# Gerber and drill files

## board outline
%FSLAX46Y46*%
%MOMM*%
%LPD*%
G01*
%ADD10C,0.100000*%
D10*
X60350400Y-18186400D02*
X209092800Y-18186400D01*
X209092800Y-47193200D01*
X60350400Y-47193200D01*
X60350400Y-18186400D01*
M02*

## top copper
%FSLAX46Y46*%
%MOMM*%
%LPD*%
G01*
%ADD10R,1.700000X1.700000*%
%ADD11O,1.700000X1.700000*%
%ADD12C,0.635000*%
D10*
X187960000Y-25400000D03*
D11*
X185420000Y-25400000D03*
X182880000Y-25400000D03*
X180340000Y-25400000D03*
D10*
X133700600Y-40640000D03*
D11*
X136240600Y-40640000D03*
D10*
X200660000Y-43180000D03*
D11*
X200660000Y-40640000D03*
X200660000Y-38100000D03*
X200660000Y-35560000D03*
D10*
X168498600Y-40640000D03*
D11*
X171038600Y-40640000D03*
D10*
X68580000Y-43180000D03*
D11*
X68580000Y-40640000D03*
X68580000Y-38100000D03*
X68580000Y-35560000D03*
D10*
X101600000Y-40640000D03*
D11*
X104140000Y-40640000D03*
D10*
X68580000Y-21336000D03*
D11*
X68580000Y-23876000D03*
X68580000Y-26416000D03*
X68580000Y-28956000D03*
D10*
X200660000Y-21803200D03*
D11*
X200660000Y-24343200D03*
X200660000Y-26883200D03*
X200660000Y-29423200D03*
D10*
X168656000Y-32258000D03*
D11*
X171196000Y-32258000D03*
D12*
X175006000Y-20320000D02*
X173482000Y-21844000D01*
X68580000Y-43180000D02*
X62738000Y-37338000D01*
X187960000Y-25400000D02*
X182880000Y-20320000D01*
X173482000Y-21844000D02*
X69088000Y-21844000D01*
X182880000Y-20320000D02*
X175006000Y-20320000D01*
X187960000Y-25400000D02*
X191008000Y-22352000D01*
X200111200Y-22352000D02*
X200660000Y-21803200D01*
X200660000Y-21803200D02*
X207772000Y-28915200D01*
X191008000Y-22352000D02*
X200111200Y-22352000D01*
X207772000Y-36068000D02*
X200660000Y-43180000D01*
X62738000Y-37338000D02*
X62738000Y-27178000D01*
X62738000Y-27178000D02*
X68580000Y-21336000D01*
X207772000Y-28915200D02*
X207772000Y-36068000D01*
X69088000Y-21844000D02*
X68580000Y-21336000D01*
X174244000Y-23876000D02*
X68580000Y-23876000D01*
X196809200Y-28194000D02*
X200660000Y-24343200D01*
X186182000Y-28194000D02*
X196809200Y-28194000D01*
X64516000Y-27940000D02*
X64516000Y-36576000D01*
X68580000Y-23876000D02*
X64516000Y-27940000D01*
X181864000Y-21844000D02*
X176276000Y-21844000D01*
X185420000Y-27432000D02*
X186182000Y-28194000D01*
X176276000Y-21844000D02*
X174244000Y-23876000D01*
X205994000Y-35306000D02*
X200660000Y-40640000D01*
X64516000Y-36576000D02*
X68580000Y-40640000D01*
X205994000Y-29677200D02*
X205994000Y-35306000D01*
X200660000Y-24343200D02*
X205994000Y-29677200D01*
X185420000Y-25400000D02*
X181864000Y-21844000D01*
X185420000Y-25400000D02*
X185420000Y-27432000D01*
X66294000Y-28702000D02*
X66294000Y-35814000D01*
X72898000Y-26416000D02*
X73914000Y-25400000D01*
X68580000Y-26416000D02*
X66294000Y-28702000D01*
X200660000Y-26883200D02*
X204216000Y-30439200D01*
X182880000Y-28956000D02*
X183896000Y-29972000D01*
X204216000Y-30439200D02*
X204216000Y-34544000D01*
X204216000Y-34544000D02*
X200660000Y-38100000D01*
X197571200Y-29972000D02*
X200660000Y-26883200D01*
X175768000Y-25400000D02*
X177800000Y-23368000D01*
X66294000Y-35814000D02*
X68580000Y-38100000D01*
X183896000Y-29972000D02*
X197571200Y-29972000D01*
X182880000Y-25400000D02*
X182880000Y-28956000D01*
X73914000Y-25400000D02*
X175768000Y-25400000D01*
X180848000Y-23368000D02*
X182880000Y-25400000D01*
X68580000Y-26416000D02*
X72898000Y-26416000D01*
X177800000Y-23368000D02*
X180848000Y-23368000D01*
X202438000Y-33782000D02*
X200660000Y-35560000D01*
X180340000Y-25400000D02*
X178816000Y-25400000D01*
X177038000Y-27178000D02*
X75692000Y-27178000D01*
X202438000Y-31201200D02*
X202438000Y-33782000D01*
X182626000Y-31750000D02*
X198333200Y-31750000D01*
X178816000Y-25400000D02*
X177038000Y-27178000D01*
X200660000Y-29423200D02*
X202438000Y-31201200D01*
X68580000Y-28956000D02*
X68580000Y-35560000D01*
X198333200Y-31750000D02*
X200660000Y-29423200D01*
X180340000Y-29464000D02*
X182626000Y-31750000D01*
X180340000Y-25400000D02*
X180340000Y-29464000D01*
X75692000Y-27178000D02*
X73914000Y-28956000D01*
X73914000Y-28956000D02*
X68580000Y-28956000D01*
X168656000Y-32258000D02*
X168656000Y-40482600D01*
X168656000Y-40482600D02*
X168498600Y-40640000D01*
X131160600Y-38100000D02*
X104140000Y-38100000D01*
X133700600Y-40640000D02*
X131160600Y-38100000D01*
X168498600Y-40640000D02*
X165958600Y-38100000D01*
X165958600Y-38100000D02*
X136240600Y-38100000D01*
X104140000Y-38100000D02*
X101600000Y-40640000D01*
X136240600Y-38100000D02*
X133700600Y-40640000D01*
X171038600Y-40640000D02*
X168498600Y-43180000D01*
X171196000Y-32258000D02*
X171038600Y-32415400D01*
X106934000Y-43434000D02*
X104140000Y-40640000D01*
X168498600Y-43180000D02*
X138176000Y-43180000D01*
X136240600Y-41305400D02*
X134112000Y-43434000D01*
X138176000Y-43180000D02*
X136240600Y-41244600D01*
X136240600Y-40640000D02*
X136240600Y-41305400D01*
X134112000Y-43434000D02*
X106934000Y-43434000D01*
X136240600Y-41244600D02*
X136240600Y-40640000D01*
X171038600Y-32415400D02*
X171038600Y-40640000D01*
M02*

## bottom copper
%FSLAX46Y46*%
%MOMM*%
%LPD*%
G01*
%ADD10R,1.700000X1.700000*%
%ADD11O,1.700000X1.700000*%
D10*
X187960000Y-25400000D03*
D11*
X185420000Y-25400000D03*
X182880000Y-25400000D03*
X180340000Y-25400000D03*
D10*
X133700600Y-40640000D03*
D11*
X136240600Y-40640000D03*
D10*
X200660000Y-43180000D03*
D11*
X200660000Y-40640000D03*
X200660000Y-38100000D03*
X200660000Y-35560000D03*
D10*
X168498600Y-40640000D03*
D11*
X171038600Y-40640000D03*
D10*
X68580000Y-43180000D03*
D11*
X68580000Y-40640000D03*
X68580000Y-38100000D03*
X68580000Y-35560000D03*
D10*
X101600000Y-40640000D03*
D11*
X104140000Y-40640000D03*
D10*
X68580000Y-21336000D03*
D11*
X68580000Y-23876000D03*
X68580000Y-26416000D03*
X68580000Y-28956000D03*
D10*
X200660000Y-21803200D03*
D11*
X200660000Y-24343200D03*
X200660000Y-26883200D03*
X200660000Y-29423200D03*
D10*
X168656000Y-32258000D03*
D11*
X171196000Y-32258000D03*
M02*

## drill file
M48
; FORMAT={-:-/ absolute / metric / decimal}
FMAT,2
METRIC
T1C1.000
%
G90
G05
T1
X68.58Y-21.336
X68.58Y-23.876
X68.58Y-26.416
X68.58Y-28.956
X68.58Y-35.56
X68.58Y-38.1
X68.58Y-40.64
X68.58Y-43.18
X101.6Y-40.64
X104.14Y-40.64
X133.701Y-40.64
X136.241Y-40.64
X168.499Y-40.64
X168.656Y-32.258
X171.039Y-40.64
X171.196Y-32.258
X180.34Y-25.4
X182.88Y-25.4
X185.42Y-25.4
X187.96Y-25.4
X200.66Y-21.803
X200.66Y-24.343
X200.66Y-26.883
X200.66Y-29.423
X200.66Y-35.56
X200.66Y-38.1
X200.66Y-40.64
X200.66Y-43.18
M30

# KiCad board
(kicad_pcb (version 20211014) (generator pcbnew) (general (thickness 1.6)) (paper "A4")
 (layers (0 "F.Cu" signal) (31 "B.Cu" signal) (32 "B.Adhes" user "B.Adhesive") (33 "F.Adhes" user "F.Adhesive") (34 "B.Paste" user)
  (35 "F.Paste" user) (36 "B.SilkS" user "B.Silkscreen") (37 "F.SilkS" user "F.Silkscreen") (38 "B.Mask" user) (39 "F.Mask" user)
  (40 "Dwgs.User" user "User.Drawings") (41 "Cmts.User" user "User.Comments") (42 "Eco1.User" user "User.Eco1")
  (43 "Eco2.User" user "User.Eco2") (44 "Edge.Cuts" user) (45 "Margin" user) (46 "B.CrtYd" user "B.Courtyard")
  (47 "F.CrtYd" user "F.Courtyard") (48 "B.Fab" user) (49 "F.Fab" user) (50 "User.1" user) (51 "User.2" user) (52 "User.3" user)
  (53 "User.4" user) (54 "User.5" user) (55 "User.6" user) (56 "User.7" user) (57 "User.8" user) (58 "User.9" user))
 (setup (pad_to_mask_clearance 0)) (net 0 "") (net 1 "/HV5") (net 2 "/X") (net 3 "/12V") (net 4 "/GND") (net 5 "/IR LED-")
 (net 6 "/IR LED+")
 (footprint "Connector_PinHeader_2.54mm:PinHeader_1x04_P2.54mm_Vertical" (layer "F.Cu") (at 187.96 25.4 -90)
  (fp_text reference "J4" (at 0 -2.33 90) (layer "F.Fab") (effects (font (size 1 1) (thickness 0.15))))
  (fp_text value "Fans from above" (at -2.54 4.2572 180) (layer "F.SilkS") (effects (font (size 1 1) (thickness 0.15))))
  (pad "1" thru_hole rect (at 0 0 270) (size 1.7 1.7) (drill 1) (layers *.Cu *.Mask) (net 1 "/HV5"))
  (pad "2" thru_hole oval (at 0 2.54 270) (size 1.7 1.7) (drill 1) (layers *.Cu *.Mask) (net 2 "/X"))
  (pad "3" thru_hole oval (at 0 5.08 270) (size 1.7 1.7) (drill 1) (layers *.Cu *.Mask) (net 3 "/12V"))
  (pad "4" thru_hole oval (at 0 7.62 270) (size 1.7 1.7) (drill 1) (layers *.Cu *.Mask) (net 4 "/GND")))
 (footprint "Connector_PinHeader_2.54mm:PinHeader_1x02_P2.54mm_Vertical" (layer "F.Cu") (at 133.7006 40.64 90)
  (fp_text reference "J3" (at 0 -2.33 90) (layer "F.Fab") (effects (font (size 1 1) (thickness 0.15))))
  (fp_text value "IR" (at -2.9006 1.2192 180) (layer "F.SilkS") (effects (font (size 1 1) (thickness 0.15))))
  (pad "1" thru_hole rect (at 0 0 90) (size 1.7 1.7) (drill 1) (layers *.Cu *.Mask) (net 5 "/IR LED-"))
  (pad "2" thru_hole oval (at 0 2.54 90) (size 1.7 1.7) (drill 1) (layers *.Cu *.Mask) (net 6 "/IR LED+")))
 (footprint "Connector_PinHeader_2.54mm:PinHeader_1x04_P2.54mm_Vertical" (layer "F.Cu") (at 200.66 43.18 180)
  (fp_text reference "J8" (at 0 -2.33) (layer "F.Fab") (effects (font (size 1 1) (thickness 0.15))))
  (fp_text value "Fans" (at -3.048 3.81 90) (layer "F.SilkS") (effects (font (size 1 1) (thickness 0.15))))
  (pad "1" thru_hole rect (at 0 0 180) (size 1.7 1.7) (drill 1) (layers *.Cu *.Mask) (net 1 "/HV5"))
  (pad "2" thru_hole oval (at 0 2.54 180) (size 1.7 1.7) (drill 1) (layers *.Cu *.Mask) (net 2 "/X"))
  (pad "3" thru_hole oval (at 0 5.08 180) (size 1.7 1.7) (drill 1) (layers *.Cu *.Mask) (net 3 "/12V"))
  (pad "4" thru_hole oval (at 0 7.62 180) (size 1.7 1.7) (drill 1) (layers *.Cu *.Mask) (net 4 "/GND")))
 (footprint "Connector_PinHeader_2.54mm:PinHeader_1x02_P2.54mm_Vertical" (layer "F.Cu") (at 168.4986 40.64 90)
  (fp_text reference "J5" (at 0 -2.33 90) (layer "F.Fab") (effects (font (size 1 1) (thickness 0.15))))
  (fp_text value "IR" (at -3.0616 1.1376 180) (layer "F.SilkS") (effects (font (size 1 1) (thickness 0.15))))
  (pad "1" thru_hole rect (at 0 0 90) (size 1.7 1.7) (drill 1) (layers *.Cu *.Mask) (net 5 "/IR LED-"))
  (pad "2" thru_hole oval (at 0 2.54 90) (size 1.7 1.7) (drill 1) (layers *.Cu *.Mask) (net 6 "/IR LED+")))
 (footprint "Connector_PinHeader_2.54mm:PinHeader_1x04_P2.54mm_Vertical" (layer "F.Cu") (at 68.58 43.18 180)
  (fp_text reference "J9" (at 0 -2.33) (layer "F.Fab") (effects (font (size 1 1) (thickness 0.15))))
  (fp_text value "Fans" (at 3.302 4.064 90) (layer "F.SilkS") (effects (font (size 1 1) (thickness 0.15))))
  (pad "1" thru_hole rect (at 0 0 180) (size 1.7 1.7) (drill 1) (layers *.Cu *.Mask) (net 1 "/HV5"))
  (pad "2" thru_hole oval (at 0 2.54 180) (size 1.7 1.7) (drill 1) (layers *.Cu *.Mask) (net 2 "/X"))
  (pad "3" thru_hole oval (at 0 5.08 180) (size 1.7 1.7) (drill 1) (layers *.Cu *.Mask) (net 3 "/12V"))
  (pad "4" thru_hole oval (at 0 7.62 180) (size 1.7 1.7) (drill 1) (layers *.Cu *.Mask) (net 4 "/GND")))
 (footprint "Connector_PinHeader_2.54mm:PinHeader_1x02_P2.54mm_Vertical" (layer "F.Cu") (at 101.6 40.64 90)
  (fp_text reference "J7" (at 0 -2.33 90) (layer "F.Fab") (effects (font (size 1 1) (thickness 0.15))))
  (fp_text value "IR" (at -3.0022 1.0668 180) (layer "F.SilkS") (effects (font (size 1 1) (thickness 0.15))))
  (pad "1" thru_hole rect (at 0 0 90) (size 1.7 1.7) (drill 1) (layers *.Cu *.Mask) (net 5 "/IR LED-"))
  (pad "2" thru_hole oval (at 0 2.54 90) (size 1.7 1.7) (drill 1) (layers *.Cu *.Mask) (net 6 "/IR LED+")))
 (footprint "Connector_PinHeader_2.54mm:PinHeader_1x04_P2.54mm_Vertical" (layer "F.Cu") (at 68.58 21.336)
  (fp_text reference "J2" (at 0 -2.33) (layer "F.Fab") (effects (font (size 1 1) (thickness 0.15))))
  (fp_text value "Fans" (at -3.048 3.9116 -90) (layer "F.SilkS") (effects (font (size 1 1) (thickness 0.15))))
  (pad "1" thru_hole rect (at 0 0) (size 1.7 1.7) (drill 1) (layers *.Cu *.Mask) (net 1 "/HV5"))
  (pad "2" thru_hole oval (at 0 2.54) (size 1.7 1.7) (drill 1) (layers *.Cu *.Mask) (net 2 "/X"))
  (pad "3" thru_hole oval (at 0 5.08) (size 1.7 1.7) (drill 1) (layers *.Cu *.Mask) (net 3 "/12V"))
  (pad "4" thru_hole oval (at 0 7.62) (size 1.7 1.7) (drill 1) (layers *.Cu *.Mask) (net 4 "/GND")))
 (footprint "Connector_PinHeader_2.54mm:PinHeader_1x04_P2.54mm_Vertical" (layer "F.Cu") (at 200.66 21.8032)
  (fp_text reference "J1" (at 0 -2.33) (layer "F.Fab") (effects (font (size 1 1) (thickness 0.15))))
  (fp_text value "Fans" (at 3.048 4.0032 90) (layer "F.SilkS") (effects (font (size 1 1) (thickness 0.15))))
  (pad "1" thru_hole rect (at 0 0) (size 1.7 1.7) (drill 1) (layers *.Cu *.Mask) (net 1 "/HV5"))
  (pad "2" thru_hole oval (at 0 2.54) (size 1.7 1.7) (drill 1) (layers *.Cu *.Mask) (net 2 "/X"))
  (pad "3" thru_hole oval (at 0 5.08) (size 1.7 1.7) (drill 1) (layers *.Cu *.Mask) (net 3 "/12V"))
  (pad "4" thru_hole oval (at 0 7.62) (size 1.7 1.7) (drill 1) (layers *.Cu *.Mask) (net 4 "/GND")))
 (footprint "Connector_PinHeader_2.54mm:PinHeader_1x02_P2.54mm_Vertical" (layer "F.Cu") (at 168.656 32.258 90)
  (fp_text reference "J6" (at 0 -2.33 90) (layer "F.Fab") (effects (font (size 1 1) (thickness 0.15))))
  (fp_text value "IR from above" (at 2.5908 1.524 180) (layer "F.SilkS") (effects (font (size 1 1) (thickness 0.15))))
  (pad "1" thru_hole rect (at 0 0 90) (size 1.7 1.7) (drill 1) (layers *.Cu *.Mask) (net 5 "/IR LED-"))
  (pad "2" thru_hole oval (at 0 2.54 90) (size 1.7 1.7) (drill 1) (layers *.Cu *.Mask) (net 6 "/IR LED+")))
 (gr_rect (start 60.3504 18.1864) (end 209.0928 47.1932) (layer "Edge.Cuts") (width 0.1) (fill none))
 (segment (start 175.006 20.32) (end 173.482 21.844) (width 0.635) (layer "F.Cu") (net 1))
 (segment (start 68.58 43.18) (end 62.738 37.338) (width 0.635) (layer "F.Cu") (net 1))
 (segment (start 187.96 25.4) (end 182.88 20.32) (width 0.635) (layer "F.Cu") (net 1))
 (segment (start 173.482 21.844) (end 69.088 21.844) (width 0.635) (layer "F.Cu") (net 1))
 (segment (start 182.88 20.32) (end 175.006 20.32) (width 0.635) (layer "F.Cu") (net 1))
 (segment (start 187.96 25.4) (end 191.008 22.352) (width 0.635) (layer "F.Cu") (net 1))
 (segment (start 200.1112 22.352) (end 200.66 21.8032) (width 0.635) (layer "F.Cu") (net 1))
 (segment (start 200.66 21.8032) (end 207.772 28.9152) (width 0.635) (layer "F.Cu") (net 1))
 (segment (start 191.008 22.352) (end 200.1112 22.352) (width 0.635) (layer "F.Cu") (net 1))
 (segment (start 207.772 36.068) (end 200.66 43.18) (width 0.635) (layer "F.Cu") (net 1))
 (segment (start 62.738 37.338) (end 62.738 27.178) (width 0.635) (layer "F.Cu") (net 1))
 (segment (start 62.738 27.178) (end 68.58 21.336) (width 0.635) (layer "F.Cu") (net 1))
 (segment (start 207.772 28.9152) (end 207.772 36.068) (width 0.635) (layer "F.Cu") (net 1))
 (segment (start 69.088 21.844) (end 68.58 21.336) (width 0.635) (layer "F.Cu") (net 1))
 (segment (start 174.244 23.876) (end 68.58 23.876) (width 0.635) (layer "F.Cu") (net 2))
 (segment (start 196.8092 28.194) (end 200.66 24.3432) (width 0.635) (layer "F.Cu") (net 2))
 (segment (start 186.182 28.194) (end 196.8092 28.194) (width 0.635) (layer "F.Cu") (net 2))
 (segment (start 64.516 27.94) (end 64.516 36.576) (width 0.635) (layer "F.Cu") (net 2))
 (segment (start 68.58 23.876) (end 64.516 27.94) (width 0.635) (layer "F.Cu") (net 2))
 (segment (start 181.864 21.844) (end 176.276 21.844) (width 0.635) (layer "F.Cu") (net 2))
 (segment (start 185.42 27.432) (end 186.182 28.194) (width 0.635) (layer "F.Cu") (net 2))
 (segment (start 176.276 21.844) (end 174.244 23.876) (width 0.635) (layer "F.Cu") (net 2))
 (segment (start 205.994 35.306) (end 200.66 40.64) (width 0.635) (layer "F.Cu") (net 2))
 (segment (start 64.516 36.576) (end 68.58 40.64) (width 0.635) (layer "F.Cu") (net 2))
 (segment (start 205.994 29.6772) (end 205.994 35.306) (width 0.635) (layer "F.Cu") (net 2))
 (segment (start 200.66 24.3432) (end 205.994 29.6772) (width 0.635) (layer "F.Cu") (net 2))
 (segment (start 185.42 25.4) (end 181.864 21.844) (width 0.635) (layer "F.Cu") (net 2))
 (segment (start 185.42 25.4) (end 185.42 27.432) (width 0.635) (layer "F.Cu") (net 2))
 (segment (start 66.294 28.702) (end 66.294 35.814) (width 0.635) (layer "F.Cu") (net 3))
 (segment (start 72.898 26.416) (end 73.914 25.4) (width 0.635) (layer "F.Cu") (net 3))
 (segment (start 68.58 26.416) (end 66.294 28.702) (width 0.635) (layer "F.Cu") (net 3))
 (segment (start 200.66 26.8832) (end 204.216 30.4392) (width 0.635) (layer "F.Cu") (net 3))
 (segment (start 182.88 28.956) (end 183.896 29.972) (width 0.635) (layer "F.Cu") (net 3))
 (segment (start 204.216 30.4392) (end 204.216 34.544) (width 0.635) (layer "F.Cu") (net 3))
 (segment (start 204.216 34.544) (end 200.66 38.1) (width 0.635) (layer "F.Cu") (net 3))
 (segment (start 197.5712 29.972) (end 200.66 26.8832) (width 0.635) (layer "F.Cu") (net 3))
 (segment (start 175.768 25.4) (end 177.8 23.368) (width 0.635) (layer "F.Cu") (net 3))
 (segment (start 66.294 35.814) (end 68.58 38.1) (width 0.635) (layer "F.Cu") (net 3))
 (segment (start 183.896 29.972) (end 197.5712 29.972) (width 0.635) (layer "F.Cu") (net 3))
 (segment (start 182.88 25.4) (end 182.88 28.956) (width 0.635) (layer "F.Cu") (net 3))
 (segment (start 73.914 25.4) (end 175.768 25.4) (width 0.635) (layer "F.Cu") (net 3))
 (segment (start 180.848 23.368) (end 182.88 25.4) (width 0.635) (layer "F.Cu") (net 3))
 (segment (start 68.58 26.416) (end 72.898 26.416) (width 0.635) (layer "F.Cu") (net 3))
 (segment (start 177.8 23.368) (end 180.848 23.368) (width 0.635) (layer "F.Cu") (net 3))
 (segment (start 202.438 33.782) (end 200.66 35.56) (width 0.635) (layer "F.Cu") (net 4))
 (segment (start 180.34 25.4) (end 178.816 25.4) (width 0.635) (layer "F.Cu") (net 4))
 (segment (start 177.038 27.178) (end 75.692 27.178) (width 0.635) (layer "F.Cu") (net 4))
 (segment (start 202.438 31.2012) (end 202.438 33.782) (width 0.635) (layer "F.Cu") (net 4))
 (segment (start 182.626 31.75) (end 198.3332 31.75) (width 0.635) (layer "F.Cu") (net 4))
 (segment (start 178.816 25.4) (end 177.038 27.178) (width 0.635) (layer "F.Cu") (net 4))
 (segment (start 200.66 29.4232) (end 202.438 31.2012) (width 0.635) (layer "F.Cu") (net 4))
 (segment (start 68.58 28.956) (end 68.58 35.56) (width 0.635) (layer "F.Cu") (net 4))
 (segment (start 198.3332 31.75) (end 200.66 29.4232) (width 0.635) (layer "F.Cu") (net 4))
 (segment (start 180.34 29.464) (end 182.626 31.75) (width 0.635) (layer "F.Cu") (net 4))
 (segment (start 180.34 25.4) (end 180.34 29.464) (width 0.635) (layer "F.Cu") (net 4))
 (segment (start 75.692 27.178) (end 73.914 28.956) (width 0.635) (layer "F.Cu") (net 4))
 (segment (start 73.914 28.956) (end 68.58 28.956) (width 0.635) (layer "F.Cu") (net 4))
 (segment (start 168.656 32.258) (end 168.656 40.4826) (width 0.635) (layer "F.Cu") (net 5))
 (segment (start 168.656 40.4826) (end 168.4986 40.64) (width 0.635) (layer "F.Cu") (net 5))
 (segment (start 131.1606 38.1) (end 104.14 38.1) (width 0.635) (layer "F.Cu") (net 5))
 (segment (start 133.7006 40.64) (end 131.1606 38.1) (width 0.635) (layer "F.Cu") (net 5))
 (segment (start 168.4986 40.64) (end 165.9586 38.1) (width 0.635) (layer "F.Cu") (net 5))
 (segment (start 165.9586 38.1) (end 136.2406 38.1) (width 0.635) (layer "F.Cu") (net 5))
 (segment (start 104.14 38.1) (end 101.6 40.64) (width 0.635) (layer "F.Cu") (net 5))
 (segment (start 136.2406 38.1) (end 133.7006 40.64) (width 0.635) (layer "F.Cu") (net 5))
 (segment (start 171.0386 40.64) (end 168.4986 43.18) (width 0.635) (layer "F.Cu") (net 6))
 (segment (start 171.196 32.258) (end 171.0386 32.4154) (width 0.635) (layer "F.Cu") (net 6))
 (segment (start 106.934 43.434) (end 104.14 40.64) (width 0.635) (layer "F.Cu") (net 6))
 (segment (start 168.4986 43.18) (end 138.176 43.18) (width 0.635) (layer "F.Cu") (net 6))
 (segment (start 136.2406 41.3054) (end 134.112 43.434) (width 0.635) (layer "F.Cu") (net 6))
 (segment (start 138.176 43.18) (end 136.2406 41.2446) (width 0.635) (layer "F.Cu") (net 6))
 (segment (start 136.2406 40.64) (end 136.2406 41.3054) (width 0.635) (layer "F.Cu") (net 6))
 (segment (start 134.112 43.434) (end 106.934 43.434) (width 0.635) (layer "F.Cu") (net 6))
 (segment (start 136.2406 41.2446) (end 136.2406 40.64) (width 0.635) (layer "F.Cu") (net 6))
 (segment (start 171.0386 32.4154) (end 171.0386 40.64) (width 0.635) (layer "F.Cu") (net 6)))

